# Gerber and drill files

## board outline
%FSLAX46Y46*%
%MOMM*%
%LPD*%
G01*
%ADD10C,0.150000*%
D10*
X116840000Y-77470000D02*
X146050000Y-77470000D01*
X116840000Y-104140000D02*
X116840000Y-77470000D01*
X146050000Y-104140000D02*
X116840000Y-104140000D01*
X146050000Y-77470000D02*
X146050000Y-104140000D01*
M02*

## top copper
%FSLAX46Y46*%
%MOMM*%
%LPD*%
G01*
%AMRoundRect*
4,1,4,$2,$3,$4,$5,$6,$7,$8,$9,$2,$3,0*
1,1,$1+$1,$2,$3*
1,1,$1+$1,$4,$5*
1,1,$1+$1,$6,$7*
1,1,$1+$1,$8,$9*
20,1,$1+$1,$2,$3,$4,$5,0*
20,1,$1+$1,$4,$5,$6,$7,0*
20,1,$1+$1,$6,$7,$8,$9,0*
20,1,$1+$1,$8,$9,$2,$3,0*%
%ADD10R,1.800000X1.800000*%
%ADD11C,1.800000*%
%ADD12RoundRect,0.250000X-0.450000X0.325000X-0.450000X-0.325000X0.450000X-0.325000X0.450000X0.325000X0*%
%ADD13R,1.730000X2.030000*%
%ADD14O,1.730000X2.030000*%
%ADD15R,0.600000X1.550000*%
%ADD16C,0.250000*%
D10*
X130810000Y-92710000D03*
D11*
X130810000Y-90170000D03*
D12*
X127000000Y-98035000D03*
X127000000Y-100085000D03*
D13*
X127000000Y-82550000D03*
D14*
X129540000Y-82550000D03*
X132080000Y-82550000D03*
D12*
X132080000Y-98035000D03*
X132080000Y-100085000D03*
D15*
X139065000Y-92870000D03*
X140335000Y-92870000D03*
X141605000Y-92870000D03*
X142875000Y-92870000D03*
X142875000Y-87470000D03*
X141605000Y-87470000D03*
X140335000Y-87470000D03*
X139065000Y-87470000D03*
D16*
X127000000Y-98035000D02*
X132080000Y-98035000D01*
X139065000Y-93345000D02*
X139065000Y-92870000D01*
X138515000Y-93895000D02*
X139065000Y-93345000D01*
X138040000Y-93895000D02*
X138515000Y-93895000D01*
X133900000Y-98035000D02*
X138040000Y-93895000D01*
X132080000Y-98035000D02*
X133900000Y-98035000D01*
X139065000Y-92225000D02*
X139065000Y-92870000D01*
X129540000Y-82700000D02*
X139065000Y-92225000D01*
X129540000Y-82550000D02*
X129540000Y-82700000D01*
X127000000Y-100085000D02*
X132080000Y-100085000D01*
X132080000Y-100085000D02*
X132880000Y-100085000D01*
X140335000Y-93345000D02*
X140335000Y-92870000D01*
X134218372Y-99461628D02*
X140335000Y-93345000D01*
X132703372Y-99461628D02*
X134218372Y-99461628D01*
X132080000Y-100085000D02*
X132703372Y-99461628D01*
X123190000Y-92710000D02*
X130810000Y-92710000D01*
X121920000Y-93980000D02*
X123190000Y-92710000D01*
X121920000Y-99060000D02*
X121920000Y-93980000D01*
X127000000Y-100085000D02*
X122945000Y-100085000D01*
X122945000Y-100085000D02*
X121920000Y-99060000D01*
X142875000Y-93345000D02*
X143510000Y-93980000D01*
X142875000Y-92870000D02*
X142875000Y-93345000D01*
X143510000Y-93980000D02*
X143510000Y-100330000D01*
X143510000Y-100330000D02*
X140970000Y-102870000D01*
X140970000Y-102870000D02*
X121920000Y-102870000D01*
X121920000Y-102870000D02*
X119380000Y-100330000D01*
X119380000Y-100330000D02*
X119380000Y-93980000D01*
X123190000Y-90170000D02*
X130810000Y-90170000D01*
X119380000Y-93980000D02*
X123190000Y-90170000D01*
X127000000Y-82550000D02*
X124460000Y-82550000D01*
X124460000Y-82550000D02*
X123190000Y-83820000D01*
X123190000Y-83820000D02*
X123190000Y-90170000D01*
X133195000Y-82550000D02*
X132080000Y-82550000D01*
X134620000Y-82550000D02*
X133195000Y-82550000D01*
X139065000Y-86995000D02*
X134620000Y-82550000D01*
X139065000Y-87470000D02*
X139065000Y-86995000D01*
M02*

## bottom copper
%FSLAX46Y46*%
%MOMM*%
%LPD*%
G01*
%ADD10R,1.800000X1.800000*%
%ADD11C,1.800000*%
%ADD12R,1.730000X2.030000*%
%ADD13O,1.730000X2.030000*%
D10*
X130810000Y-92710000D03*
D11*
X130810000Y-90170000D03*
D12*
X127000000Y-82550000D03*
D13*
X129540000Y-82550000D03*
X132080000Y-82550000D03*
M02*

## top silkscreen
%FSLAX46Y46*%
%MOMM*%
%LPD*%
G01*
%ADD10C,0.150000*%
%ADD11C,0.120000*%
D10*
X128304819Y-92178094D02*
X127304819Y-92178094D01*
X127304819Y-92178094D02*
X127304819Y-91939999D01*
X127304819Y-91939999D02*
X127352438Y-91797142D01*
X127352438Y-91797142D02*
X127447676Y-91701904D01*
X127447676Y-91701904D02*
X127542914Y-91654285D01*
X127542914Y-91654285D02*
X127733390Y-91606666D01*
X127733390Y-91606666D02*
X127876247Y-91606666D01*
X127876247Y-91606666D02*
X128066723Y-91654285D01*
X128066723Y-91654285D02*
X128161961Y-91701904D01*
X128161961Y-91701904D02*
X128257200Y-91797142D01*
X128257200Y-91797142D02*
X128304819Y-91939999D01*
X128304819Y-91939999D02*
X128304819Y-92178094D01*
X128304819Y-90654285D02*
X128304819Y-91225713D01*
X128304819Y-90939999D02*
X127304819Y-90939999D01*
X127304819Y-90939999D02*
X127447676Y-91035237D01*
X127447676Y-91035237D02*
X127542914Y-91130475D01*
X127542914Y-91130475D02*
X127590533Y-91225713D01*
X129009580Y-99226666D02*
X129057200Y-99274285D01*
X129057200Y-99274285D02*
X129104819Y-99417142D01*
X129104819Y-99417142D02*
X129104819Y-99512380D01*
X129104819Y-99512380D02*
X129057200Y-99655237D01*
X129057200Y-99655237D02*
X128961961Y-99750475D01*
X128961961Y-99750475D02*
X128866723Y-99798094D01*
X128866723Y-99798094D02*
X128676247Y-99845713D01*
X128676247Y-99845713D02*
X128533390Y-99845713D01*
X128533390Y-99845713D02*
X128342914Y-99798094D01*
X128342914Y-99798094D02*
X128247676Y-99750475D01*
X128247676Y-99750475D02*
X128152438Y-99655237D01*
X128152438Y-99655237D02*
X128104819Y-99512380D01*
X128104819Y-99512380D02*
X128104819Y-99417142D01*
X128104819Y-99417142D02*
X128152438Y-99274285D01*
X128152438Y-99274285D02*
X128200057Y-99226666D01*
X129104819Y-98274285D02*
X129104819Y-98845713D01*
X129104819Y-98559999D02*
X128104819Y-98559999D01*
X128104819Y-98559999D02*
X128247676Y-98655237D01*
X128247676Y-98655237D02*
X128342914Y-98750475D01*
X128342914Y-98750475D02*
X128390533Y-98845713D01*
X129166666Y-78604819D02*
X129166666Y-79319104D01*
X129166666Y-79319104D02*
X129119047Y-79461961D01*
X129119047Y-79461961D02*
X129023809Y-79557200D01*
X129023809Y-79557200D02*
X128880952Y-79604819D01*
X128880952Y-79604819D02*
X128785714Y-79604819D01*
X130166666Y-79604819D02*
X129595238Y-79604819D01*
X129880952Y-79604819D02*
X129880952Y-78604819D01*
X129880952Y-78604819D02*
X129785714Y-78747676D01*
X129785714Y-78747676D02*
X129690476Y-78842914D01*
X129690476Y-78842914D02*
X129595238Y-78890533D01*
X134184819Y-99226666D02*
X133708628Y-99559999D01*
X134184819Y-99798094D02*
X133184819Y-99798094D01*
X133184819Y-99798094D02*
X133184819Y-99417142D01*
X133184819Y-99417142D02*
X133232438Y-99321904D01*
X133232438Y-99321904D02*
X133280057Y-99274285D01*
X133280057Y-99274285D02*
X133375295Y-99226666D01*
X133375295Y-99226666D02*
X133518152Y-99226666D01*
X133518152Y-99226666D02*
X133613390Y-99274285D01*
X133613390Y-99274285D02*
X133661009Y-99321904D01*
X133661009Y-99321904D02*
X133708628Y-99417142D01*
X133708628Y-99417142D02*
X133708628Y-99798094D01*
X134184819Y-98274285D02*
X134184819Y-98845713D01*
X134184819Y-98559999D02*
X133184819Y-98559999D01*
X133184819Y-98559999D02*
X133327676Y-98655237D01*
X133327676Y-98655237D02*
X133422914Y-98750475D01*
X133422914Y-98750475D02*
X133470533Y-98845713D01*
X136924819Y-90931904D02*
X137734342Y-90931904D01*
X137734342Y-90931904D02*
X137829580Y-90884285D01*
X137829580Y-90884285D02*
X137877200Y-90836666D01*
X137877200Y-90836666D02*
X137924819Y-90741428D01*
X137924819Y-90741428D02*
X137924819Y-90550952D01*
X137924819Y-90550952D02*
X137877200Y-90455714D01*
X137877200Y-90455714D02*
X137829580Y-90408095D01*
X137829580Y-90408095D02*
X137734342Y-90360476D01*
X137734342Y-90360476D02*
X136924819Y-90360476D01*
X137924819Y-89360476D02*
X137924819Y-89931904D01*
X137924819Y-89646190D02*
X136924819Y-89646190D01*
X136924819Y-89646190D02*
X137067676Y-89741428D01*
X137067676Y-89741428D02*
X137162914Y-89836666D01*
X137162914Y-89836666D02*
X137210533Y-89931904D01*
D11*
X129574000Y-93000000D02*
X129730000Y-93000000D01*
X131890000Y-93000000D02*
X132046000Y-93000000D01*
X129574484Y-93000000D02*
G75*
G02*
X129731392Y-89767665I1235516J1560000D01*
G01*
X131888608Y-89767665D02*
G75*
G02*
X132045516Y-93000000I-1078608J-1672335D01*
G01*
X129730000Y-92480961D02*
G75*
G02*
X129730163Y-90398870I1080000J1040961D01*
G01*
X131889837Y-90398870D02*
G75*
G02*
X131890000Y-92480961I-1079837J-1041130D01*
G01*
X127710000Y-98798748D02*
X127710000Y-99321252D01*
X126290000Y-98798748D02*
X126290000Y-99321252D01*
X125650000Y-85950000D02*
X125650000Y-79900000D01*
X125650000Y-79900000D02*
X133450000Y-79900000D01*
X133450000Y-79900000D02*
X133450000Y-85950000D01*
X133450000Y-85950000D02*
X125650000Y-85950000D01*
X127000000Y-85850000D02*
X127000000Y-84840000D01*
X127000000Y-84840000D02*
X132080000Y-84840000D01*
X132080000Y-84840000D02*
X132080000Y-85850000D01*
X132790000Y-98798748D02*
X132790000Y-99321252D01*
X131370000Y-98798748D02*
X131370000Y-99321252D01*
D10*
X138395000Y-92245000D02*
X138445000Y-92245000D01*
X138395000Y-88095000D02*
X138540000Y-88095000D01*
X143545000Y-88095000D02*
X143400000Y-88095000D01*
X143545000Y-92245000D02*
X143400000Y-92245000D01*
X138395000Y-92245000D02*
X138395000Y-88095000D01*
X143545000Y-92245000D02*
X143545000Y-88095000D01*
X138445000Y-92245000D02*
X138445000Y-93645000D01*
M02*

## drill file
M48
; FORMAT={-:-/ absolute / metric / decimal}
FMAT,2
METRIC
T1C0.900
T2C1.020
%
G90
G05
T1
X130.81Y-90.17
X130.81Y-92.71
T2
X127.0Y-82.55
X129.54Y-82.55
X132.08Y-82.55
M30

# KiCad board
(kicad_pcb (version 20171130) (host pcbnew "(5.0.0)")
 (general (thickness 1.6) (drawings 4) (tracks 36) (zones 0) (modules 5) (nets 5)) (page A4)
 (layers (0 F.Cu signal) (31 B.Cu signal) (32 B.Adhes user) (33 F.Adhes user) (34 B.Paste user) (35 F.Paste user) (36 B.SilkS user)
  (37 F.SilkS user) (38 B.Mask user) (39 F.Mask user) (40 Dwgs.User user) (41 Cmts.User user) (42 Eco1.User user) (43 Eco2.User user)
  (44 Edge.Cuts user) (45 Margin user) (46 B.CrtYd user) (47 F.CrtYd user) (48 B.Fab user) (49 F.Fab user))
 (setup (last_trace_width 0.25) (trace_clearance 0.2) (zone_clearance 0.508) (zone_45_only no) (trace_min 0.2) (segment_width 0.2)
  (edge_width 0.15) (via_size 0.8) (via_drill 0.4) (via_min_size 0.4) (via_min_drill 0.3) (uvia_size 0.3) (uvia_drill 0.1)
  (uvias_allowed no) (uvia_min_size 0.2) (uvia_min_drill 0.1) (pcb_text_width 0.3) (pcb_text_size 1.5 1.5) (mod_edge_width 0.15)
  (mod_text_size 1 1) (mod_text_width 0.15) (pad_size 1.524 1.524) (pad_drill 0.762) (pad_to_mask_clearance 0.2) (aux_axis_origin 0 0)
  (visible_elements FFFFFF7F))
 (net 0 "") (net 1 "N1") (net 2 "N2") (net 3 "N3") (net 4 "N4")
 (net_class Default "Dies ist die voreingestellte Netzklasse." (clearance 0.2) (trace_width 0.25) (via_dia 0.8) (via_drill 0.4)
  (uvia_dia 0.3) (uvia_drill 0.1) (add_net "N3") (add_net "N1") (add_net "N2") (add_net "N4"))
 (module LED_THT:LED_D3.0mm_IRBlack (layer F.Cu) (at 130.81 92.71 90)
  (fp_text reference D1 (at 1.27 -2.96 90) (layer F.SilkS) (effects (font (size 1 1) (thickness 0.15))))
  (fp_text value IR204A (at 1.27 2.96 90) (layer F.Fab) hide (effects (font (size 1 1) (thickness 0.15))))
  (fp_line (start -0.29 -1.236) (end -0.29 -1.08) (layer F.SilkS) (width 0.12))
  (fp_line (start -0.29 1.08) (end -0.29 1.236) (layer F.SilkS) (width 0.12))
  (fp_arc (start 1.27 0) (end -0.29 -1.235516) (angle 108.8) (layer F.SilkS) (width 0.12))
  (fp_arc (start 1.27 0) (end -0.29 1.235516) (angle -108.8) (layer F.SilkS) (width 0.12))
  (fp_arc (start 1.27 0) (end 0.229039 -1.08) (angle 87.9) (layer F.SilkS) (width 0.12))
  (fp_arc (start 1.27 0) (end 0.229039 1.08) (angle -87.9) (layer F.SilkS) (width 0.12))
  (pad 1 thru_hole rect (at 0 0 90) (size 1.8 1.8) (drill 0.9) (layers *.Cu *.Mask) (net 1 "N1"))
  (pad 2 thru_hole circle (at 2.54 0 90) (size 1.8 1.8) (drill 0.9) (layers *.Cu *.Mask) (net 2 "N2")))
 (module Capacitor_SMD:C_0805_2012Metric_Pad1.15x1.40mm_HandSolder (layer F.Cu) (at 127 99.06 270)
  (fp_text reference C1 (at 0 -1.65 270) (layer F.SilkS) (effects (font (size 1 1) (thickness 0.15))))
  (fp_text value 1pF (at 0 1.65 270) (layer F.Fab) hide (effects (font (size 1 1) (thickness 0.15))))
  (fp_line (start -0.261252 -0.71) (end 0.261252 -0.71) (layer F.SilkS) (width 0.12))
  (fp_line (start -0.261252 0.71) (end 0.261252 0.71) (layer F.SilkS) (width 0.12))
  (pad 1 smd roundrect (at -1.025 0 270) (size 1.15 1.4) (layers F.Cu F.Paste F.Mask) (roundrect_rratio 0.217391) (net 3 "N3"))
  (pad 2 smd roundrect (at 1.025 0 270) (size 1.15 1.4) (layers F.Cu F.Paste F.Mask) (roundrect_rratio 0.217391) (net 1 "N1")))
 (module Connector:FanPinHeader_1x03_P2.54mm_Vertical (layer F.Cu) (at 127 82.55)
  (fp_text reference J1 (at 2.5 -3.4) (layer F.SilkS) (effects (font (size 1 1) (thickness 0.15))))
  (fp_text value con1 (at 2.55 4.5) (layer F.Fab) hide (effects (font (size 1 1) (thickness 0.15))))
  (fp_line (start -1.35 3.4) (end -1.35 -2.65) (layer F.SilkS) (width 0.12))
  (fp_line (start -1.35 -2.65) (end 6.45 -2.65) (layer F.SilkS) (width 0.12))
  (fp_line (start 6.45 -2.65) (end 6.45 3.4) (layer F.SilkS) (width 0.12))
  (fp_line (start 6.45 3.4) (end -1.35 3.4) (layer F.SilkS) (width 0.12))
  (fp_line (start 0 3.3) (end 0 2.29) (layer F.SilkS) (width 0.12))
  (fp_line (start 0 2.29) (end 5.08 2.29) (layer F.SilkS) (width 0.12))
  (fp_line (start 5.08 2.29) (end 5.08 3.3) (layer F.SilkS) (width 0.12))
  (pad 1 thru_hole rect (at 0 0 90) (size 2.03 1.73) (drill 1.02) (layers *.Cu *.Mask) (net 2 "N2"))
  (pad 2 thru_hole oval (at 2.54 0 90) (size 2.03 1.73) (drill 1.02) (layers *.Cu *.Mask) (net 3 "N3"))
  (pad 3 thru_hole oval (at 5.08 0 90) (size 2.03 1.73) (drill 1.02) (layers *.Cu *.Mask) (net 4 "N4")))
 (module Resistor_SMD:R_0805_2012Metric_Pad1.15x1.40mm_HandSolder (layer F.Cu) (at 132.08 99.06 270)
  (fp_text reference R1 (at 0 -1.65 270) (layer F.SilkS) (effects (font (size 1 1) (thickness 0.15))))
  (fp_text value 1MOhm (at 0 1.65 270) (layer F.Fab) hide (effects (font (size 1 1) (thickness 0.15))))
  (fp_line (start -0.261252 -0.71) (end 0.261252 -0.71) (layer F.SilkS) (width 0.12))
  (fp_line (start -0.261252 0.71) (end 0.261252 0.71) (layer F.SilkS) (width 0.12))
  (pad 1 smd roundrect (at -1.025 0 270) (size 1.15 1.4) (layers F.Cu F.Paste F.Mask) (roundrect_rratio 0.217391) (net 3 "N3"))
  (pad 2 smd roundrect (at 1.025 0 270) (size 1.15 1.4) (layers F.Cu F.Paste F.Mask) (roundrect_rratio 0.217391) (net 1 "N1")))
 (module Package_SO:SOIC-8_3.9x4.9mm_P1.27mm (layer F.Cu) (at 140.97 90.17 90)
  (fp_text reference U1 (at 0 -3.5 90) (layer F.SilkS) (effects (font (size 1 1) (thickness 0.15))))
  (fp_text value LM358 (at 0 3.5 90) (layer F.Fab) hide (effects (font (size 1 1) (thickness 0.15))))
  (fp_line (start -2.075 -2.575) (end -2.075 -2.525) (layer F.SilkS) (width 0.15))
  (fp_line (start 2.075 -2.575) (end 2.075 -2.43) (layer F.SilkS) (width 0.15))
  (fp_line (start 2.075 2.575) (end 2.075 2.43) (layer F.SilkS) (width 0.15))
  (fp_line (start -2.075 2.575) (end -2.075 2.43) (layer F.SilkS) (width 0.15))
  (fp_line (start -2.075 -2.575) (end 2.075 -2.575) (layer F.SilkS) (width 0.15))
  (fp_line (start -2.075 2.575) (end 2.075 2.575) (layer F.SilkS) (width 0.15))
  (fp_line (start -2.075 -2.525) (end -3.475 -2.525) (layer F.SilkS) (width 0.15))
  (pad 1 smd rect (at -2.7 -1.905 90) (size 1.55 0.6) (layers F.Cu F.Paste F.Mask) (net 3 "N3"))
  (pad 2 smd rect (at -2.7 -0.635 90) (size 1.55 0.6) (layers F.Cu F.Paste F.Mask) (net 1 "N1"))
  (pad 3 smd rect (at -2.7 0.635 90) (size 1.55 0.6) (layers F.Cu F.Paste F.Mask) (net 2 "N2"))
  (pad 4 smd rect (at -2.7 1.905 90) (size 1.55 0.6) (layers F.Cu F.Paste F.Mask) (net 2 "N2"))
  (pad 5 smd rect (at 2.7 1.905 90) (size 1.55 0.6) (layers F.Cu F.Paste F.Mask))
  (pad 6 smd rect (at 2.7 0.635 90) (size 1.55 0.6) (layers F.Cu F.Paste F.Mask))
  (pad 7 smd rect (at 2.7 -0.635 90) (size 1.55 0.6) (layers F.Cu F.Paste F.Mask))
  (pad 8 smd rect (at 2.7 -1.905 90) (size 1.55 0.6) (layers F.Cu F.Paste F.Mask) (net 4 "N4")))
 (gr_line (start 116.84 77.47) (end 146.05 77.47) (layer Edge.Cuts) (width 0.15))
 (gr_line (start 116.84 104.14) (end 116.84 77.47) (layer Edge.Cuts) (width 0.15))
 (gr_line (start 146.05 104.14) (end 116.84 104.14) (layer Edge.Cuts) (width 0.15))
 (gr_line (start 146.05 77.47) (end 146.05 104.14) (layer Edge.Cuts) (width 0.15))
 (segment (start 127 98.035) (end 132.08 98.035) (width 0.25) (layer F.Cu) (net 3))
 (segment (start 139.065 93.345) (end 139.065 92.87) (width 0.25) (layer F.Cu) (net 3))
 (segment (start 138.515 93.895) (end 139.065 93.345) (width 0.25) (layer F.Cu) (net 3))
 (segment (start 138.04 93.895) (end 138.515 93.895) (width 0.25) (layer F.Cu) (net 3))
 (segment (start 133.9 98.035) (end 138.04 93.895) (width 0.25) (layer F.Cu) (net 3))
 (segment (start 132.08 98.035) (end 133.9 98.035) (width 0.25) (layer F.Cu) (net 3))
 (segment (start 139.065 92.225) (end 139.065 92.87) (width 0.25) (layer F.Cu) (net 3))
 (segment (start 129.54 82.7) (end 139.065 92.225) (width 0.25) (layer F.Cu) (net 3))
 (segment (start 129.54 82.55) (end 129.54 82.7) (width 0.25) (layer F.Cu) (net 3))
 (segment (start 127 100.085) (end 132.08 100.085) (width 0.25) (layer F.Cu) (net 1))
 (segment (start 132.08 100.085) (end 132.88 100.085) (width 0.25) (layer F.Cu) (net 1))
 (segment (start 140.335 93.345) (end 140.335 92.87) (width 0.25) (layer F.Cu) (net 1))
 (segment (start 134.218372 99.461628) (end 140.335 93.345) (width 0.25) (layer F.Cu) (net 1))
 (segment (start 132.703372 99.461628) (end 134.218372 99.461628) (width 0.25) (layer F.Cu) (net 1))
 (segment (start 132.08 100.085) (end 132.703372 99.461628) (width 0.25) (layer F.Cu) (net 1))
 (segment (start 123.19 92.71) (end 130.81 92.71) (width 0.25) (layer F.Cu) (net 1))
 (segment (start 121.92 93.98) (end 123.19 92.71) (width 0.25) (layer F.Cu) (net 1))
 (segment (start 121.92 99.06) (end 121.92 93.98) (width 0.25) (layer F.Cu) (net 1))
 (segment (start 127 100.085) (end 122.945 100.085) (width 0.25) (layer F.Cu) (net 1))
 (segment (start 122.945 100.085) (end 121.92 99.06) (width 0.25) (layer F.Cu) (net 1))
 (segment (start 142.875 93.345) (end 143.51 93.98) (width 0.25) (layer F.Cu) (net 2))
 (segment (start 142.875 92.87) (end 142.875 93.345) (width 0.25) (layer F.Cu) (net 2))
 (segment (start 143.51 93.98) (end 143.51 100.33) (width 0.25) (layer F.Cu) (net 2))
 (segment (start 143.51 100.33) (end 140.97 102.87) (width 0.25) (layer F.Cu) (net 2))
 (segment (start 140.97 102.87) (end 121.92 102.87) (width 0.25) (layer F.Cu) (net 2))
 (segment (start 121.92 102.87) (end 119.38 100.33) (width 0.25) (layer F.Cu) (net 2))
 (segment (start 119.38 100.33) (end 119.38 93.98) (width 0.25) (layer F.Cu) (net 2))
 (segment (start 123.19 90.17) (end 130.81 90.17) (width 0.25) (layer F.Cu) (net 2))
 (segment (start 119.38 93.98) (end 123.19 90.17) (width 0.25) (layer F.Cu) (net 2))
 (segment (start 127 82.55) (end 124.46 82.55) (width 0.25) (layer F.Cu) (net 2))
 (segment (start 124.46 82.55) (end 123.19 83.82) (width 0.25) (layer F.Cu) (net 2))
 (segment (start 123.19 83.82) (end 123.19 90.17) (width 0.25) (layer F.Cu) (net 2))
 (segment (start 133.195 82.55) (end 132.08 82.55) (width 0.25) (layer F.Cu) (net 4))
 (segment (start 134.62 82.55) (end 133.195 82.55) (width 0.25) (layer F.Cu) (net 4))
 (segment (start 139.065 86.995) (end 134.62 82.55) (width 0.25) (layer F.Cu) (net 4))
 (segment (start 139.065 87.47) (end 139.065 86.995) (width 0.25) (layer F.Cu) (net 4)))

